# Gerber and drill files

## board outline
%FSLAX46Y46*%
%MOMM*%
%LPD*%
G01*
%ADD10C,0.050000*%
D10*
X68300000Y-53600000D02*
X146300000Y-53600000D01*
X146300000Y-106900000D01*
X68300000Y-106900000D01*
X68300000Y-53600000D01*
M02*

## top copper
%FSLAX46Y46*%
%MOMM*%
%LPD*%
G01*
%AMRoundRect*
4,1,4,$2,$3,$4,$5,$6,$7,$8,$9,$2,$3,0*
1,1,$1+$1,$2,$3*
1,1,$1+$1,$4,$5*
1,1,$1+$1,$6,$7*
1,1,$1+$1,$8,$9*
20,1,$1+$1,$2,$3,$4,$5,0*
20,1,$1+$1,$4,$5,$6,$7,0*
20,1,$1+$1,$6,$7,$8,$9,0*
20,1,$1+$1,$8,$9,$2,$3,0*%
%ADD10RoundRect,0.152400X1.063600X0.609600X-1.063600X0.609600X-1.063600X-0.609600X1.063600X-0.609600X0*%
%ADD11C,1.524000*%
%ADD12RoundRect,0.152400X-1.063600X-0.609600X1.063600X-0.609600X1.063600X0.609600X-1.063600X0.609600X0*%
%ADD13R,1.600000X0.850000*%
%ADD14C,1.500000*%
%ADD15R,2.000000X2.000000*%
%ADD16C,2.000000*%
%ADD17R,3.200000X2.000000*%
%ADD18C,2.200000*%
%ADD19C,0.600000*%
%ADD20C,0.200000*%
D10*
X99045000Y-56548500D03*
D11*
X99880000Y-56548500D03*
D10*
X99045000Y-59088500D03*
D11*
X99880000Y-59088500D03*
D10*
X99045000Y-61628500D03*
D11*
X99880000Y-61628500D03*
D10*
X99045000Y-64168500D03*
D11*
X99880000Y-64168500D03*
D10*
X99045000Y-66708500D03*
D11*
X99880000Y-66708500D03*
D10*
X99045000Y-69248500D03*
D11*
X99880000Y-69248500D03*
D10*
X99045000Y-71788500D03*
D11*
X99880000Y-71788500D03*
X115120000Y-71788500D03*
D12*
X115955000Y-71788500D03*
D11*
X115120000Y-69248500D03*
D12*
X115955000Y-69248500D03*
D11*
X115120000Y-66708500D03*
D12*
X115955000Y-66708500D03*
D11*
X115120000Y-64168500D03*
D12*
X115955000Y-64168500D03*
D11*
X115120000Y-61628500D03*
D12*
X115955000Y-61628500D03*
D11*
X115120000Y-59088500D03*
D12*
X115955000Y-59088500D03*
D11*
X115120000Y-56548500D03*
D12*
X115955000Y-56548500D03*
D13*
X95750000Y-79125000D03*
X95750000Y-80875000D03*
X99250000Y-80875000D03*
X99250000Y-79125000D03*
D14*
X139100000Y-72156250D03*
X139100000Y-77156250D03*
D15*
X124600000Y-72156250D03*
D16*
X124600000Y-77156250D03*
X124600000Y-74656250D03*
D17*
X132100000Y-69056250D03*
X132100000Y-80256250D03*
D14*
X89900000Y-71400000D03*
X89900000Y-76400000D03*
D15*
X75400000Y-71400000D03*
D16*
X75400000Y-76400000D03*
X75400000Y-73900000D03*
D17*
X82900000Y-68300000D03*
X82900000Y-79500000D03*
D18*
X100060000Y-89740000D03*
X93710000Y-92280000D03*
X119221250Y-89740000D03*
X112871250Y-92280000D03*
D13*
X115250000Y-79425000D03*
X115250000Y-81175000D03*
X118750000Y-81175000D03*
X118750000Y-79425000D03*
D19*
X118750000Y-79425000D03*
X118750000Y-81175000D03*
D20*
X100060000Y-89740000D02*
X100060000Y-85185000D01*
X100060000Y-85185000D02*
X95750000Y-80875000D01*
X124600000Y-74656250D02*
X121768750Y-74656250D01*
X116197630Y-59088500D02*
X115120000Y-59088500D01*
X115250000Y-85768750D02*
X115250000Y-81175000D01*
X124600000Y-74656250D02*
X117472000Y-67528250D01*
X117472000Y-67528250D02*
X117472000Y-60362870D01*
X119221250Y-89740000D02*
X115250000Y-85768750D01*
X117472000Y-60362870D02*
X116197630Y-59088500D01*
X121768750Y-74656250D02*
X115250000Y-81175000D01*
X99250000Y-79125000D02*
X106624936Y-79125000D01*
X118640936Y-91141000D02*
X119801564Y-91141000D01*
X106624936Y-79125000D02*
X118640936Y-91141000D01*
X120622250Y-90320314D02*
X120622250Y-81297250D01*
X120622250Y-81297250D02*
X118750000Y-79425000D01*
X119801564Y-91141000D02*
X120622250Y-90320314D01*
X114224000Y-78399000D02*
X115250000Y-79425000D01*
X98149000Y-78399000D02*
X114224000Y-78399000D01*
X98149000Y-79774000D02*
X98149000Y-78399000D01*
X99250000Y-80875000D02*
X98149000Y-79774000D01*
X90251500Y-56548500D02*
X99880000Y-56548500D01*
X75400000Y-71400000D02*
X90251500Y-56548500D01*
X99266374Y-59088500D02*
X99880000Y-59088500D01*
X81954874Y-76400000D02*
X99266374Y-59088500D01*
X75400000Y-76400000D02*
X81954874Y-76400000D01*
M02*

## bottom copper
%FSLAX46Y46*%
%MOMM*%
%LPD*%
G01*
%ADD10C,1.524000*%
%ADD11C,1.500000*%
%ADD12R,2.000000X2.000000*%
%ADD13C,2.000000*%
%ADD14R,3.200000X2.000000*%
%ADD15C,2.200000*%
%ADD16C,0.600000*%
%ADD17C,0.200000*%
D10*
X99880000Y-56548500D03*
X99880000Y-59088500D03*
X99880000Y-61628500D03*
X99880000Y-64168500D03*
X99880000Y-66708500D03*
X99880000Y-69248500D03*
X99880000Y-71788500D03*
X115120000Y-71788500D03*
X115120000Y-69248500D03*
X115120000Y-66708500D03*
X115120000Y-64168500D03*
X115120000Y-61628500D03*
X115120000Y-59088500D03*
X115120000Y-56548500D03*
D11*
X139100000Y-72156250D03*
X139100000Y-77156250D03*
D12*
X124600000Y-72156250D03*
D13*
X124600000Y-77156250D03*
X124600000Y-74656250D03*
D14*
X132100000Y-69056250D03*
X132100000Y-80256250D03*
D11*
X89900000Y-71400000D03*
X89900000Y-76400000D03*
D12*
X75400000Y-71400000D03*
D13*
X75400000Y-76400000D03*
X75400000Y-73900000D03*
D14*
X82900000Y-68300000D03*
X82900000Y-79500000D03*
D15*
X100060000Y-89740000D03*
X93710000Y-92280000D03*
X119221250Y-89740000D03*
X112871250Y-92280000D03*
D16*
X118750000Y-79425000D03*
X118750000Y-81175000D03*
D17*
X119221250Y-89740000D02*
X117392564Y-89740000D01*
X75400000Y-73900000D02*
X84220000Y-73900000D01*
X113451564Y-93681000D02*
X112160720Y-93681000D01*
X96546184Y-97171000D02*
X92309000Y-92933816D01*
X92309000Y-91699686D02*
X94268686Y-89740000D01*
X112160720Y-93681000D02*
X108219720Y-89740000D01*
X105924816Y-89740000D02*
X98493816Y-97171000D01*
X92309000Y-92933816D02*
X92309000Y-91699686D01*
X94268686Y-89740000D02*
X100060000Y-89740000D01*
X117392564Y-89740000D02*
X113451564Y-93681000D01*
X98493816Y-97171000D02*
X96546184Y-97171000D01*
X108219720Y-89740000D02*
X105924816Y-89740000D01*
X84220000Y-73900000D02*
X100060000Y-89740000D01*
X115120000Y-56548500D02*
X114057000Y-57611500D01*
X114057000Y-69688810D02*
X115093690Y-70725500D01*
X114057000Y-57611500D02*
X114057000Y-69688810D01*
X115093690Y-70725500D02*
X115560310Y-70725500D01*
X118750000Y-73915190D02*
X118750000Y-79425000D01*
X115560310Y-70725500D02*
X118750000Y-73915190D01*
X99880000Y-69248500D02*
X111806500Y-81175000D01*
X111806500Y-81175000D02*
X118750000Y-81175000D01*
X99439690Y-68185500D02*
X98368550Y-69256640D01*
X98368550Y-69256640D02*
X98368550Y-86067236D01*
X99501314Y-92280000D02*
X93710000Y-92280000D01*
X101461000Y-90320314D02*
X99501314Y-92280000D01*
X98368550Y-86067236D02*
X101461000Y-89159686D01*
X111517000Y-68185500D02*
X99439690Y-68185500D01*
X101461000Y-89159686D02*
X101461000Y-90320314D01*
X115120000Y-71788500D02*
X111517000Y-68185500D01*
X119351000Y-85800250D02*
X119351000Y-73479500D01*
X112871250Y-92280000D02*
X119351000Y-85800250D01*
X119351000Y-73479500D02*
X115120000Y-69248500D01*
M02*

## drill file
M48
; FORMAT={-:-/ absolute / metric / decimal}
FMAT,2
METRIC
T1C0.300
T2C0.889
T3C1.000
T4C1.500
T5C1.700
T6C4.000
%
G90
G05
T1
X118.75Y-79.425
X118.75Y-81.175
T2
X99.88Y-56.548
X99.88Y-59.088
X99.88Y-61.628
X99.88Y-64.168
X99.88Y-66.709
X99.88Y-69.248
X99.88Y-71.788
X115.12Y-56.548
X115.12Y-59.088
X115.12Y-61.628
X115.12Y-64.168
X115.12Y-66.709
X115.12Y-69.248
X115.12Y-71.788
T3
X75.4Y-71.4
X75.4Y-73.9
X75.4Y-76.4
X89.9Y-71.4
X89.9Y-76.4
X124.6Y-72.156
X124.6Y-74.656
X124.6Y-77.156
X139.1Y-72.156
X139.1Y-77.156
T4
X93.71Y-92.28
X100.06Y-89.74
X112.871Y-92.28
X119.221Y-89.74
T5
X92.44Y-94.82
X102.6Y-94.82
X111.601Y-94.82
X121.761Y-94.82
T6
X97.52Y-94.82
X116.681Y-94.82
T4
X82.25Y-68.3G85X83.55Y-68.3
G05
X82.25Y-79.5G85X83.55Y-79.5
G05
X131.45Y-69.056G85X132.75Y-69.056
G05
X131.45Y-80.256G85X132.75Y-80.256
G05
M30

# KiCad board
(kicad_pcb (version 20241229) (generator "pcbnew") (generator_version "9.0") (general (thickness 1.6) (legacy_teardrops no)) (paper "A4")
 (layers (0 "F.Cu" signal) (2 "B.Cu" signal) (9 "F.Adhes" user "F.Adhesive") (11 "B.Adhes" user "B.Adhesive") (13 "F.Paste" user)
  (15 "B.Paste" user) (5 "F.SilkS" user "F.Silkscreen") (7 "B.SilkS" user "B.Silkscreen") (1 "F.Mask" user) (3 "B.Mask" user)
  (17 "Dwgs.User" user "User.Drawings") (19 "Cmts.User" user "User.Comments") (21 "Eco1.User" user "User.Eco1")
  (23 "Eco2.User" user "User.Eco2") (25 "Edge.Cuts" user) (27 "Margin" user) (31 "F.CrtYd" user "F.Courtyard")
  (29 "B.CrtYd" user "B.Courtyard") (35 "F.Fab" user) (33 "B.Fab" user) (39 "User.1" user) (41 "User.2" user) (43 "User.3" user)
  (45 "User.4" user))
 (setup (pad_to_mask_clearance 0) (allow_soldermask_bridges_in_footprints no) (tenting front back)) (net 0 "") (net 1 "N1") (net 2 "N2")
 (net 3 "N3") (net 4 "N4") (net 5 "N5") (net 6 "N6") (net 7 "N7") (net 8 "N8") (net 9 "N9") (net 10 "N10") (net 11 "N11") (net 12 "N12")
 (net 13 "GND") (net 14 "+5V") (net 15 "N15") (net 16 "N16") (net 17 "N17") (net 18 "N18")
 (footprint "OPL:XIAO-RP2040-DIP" (layer "F.Cu") (at 107.5 64.1685)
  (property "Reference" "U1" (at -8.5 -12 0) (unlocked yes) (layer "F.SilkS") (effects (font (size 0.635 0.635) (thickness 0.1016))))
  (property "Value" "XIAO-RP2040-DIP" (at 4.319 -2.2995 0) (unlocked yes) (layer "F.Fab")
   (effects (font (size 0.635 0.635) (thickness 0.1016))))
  (pad "1" smd roundrect (at -8.455 -7.62 180) (size 2.432 1.524) (layers "F.Cu" "F.Mask") (roundrect_rratio 0.1) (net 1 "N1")
   (thermal_bridge_angle 45))
  (pad "1" thru_hole circle (at -7.62 -7.62 180) (size 1.524 1.524) (drill 0.889) (layers "*.Cu" "*.Mask") (remove_unused_layers no)
   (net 1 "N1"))
  (pad "2" smd roundrect (at -8.455 -5.08 180) (size 2.432 1.524) (layers "F.Cu" "F.Mask") (roundrect_rratio 0.1) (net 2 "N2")
   (thermal_bridge_angle 45))
  (pad "2" thru_hole circle (at -7.62 -5.08 180) (size 1.524 1.524) (drill 0.889) (layers "*.Cu" "*.Mask") (remove_unused_layers no)
   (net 2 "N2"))
  (pad "3" smd roundrect (at -8.455 -2.54 180) (size 2.432 1.524) (layers "F.Cu" "F.Mask") (roundrect_rratio 0.1) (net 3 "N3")
   (thermal_bridge_angle 45))
  (pad "3" thru_hole circle (at -7.62 -2.54 180) (size 1.524 1.524) (drill 0.889) (layers "*.Cu" "*.Mask") (remove_unused_layers no)
   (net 3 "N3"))
  (pad "4" smd roundrect (at -8.455 0 180) (size 2.432 1.524) (layers "F.Cu" "F.Mask") (roundrect_rratio 0.1) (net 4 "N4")
   (thermal_bridge_angle 45))
  (pad "4" thru_hole circle (at -7.62 0 180) (size 1.524 1.524) (drill 0.889) (layers "*.Cu" "*.Mask") (remove_unused_layers no)
   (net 4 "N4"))
  (pad "5" smd roundrect (at -8.455 2.54 180) (size 2.432 1.524) (layers "F.Cu" "F.Mask") (roundrect_rratio 0.1) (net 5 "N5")
   (thermal_bridge_angle 45))
  (pad "5" thru_hole circle (at -7.62 2.54 180) (size 1.524 1.524) (drill 0.889) (layers "*.Cu" "*.Mask") (remove_unused_layers no)
   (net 5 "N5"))
  (pad "6" smd roundrect (at -8.455 5.08 180) (size 2.432 1.524) (layers "F.Cu" "F.Mask") (roundrect_rratio 0.1) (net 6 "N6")
   (thermal_bridge_angle 45))
  (pad "6" thru_hole circle (at -7.62 5.08 180) (size 1.524 1.524) (drill 0.889) (layers "*.Cu" "*.Mask") (remove_unused_layers no)
   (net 6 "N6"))
  (pad "7" smd roundrect (at -8.455 7.62 180) (size 2.432 1.524) (layers "F.Cu" "F.Mask") (roundrect_rratio 0.1) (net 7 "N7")
   (thermal_bridge_angle 45))
  (pad "7" thru_hole circle (at -7.62 7.62 180) (size 1.524 1.524) (drill 0.889) (layers "*.Cu" "*.Mask") (remove_unused_layers no)
   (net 7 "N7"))
  (pad "8" thru_hole circle (at 7.62 7.62) (size 1.524 1.524) (drill 0.889) (layers "*.Cu" "*.Mask") (remove_unused_layers no) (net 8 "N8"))
  (pad "8" smd roundrect (at 8.455 7.62) (size 2.432 1.524) (layers "F.Cu" "F.Mask") (roundrect_rratio 0.1) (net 8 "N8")
   (thermal_bridge_angle 45))
  (pad "9" thru_hole circle (at 7.62 5.08) (size 1.524 1.524) (drill 0.889) (layers "*.Cu" "*.Mask") (remove_unused_layers no) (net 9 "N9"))
  (pad "9" smd roundrect (at 8.455 5.08) (size 2.432 1.524) (layers "F.Cu" "F.Mask") (roundrect_rratio 0.1) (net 9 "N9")
   (thermal_bridge_angle 45))
  (pad "10" thru_hole circle (at 7.62 2.54) (size 1.524 1.524) (drill 0.889) (layers "*.Cu" "*.Mask") (remove_unused_layers no)
   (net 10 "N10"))
  (pad "10" smd roundrect (at 8.455 2.54) (size 2.432 1.524) (layers "F.Cu" "F.Mask") (roundrect_rratio 0.1) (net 10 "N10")
   (thermal_bridge_angle 45))
  (pad "11" thru_hole circle (at 7.62 0) (size 1.524 1.524) (drill 0.889) (layers "*.Cu" "*.Mask") (remove_unused_layers no) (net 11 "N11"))
  (pad "11" smd roundrect (at 8.455 0) (size 2.432 1.524) (layers "F.Cu" "F.Mask") (roundrect_rratio 0.1) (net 11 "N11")
   (thermal_bridge_angle 45))
  (pad "12" thru_hole circle (at 7.62 -2.54) (size 1.524 1.524) (drill 0.889) (layers "*.Cu" "*.Mask") (remove_unused_layers no)
   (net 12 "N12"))
  (pad "12" smd roundrect (at 8.455 -2.54) (size 2.432 1.524) (layers "F.Cu" "F.Mask") (roundrect_rratio 0.1) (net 12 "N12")
   (thermal_bridge_angle 45))
  (pad "13" thru_hole circle (at 7.62 -5.08) (size 1.524 1.524) (drill 0.889) (layers "*.Cu" "*.Mask") (remove_unused_layers no)
   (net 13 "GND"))
  (pad "13" smd roundrect (at 8.455 -5.08) (size 2.432 1.524) (layers "F.Cu" "F.Mask") (roundrect_rratio 0.1) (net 13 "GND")
   (thermal_bridge_angle 45))
  (pad "14" thru_hole circle (at 7.62 -7.62) (size 1.524 1.524) (drill 0.889) (layers "*.Cu" "*.Mask") (remove_unused_layers no)
   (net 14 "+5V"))
  (pad "14" smd roundrect (at 8.455 -7.62) (size 2.432 1.524) (layers "F.Cu" "F.Mask") (roundrect_rratio 0.1) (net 14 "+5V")
   (thermal_bridge_angle 45)))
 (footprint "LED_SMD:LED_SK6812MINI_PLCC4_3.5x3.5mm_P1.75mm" (layer "F.Cu") (at 97.5 80)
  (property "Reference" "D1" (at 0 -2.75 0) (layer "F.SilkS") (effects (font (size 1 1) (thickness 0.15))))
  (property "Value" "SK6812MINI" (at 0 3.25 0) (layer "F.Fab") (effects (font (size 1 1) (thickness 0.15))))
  (pad "1" smd rect (at -1.75 -0.875) (size 1.6 0.85) (layers "F.Cu" "F.Mask" "F.Paste") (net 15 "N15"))
  (pad "2" smd rect (at -1.75 0.875) (size 1.6 0.85) (layers "F.Cu" "F.Mask" "F.Paste") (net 13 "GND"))
  (pad "3" smd rect (at 1.75 0.875) (size 1.6 0.85) (layers "F.Cu" "F.Mask" "F.Paste") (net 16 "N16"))
  (pad "4" smd rect (at 1.75 -0.875) (size 1.6 0.85) (layers "F.Cu" "F.Mask" "F.Paste") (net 14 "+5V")))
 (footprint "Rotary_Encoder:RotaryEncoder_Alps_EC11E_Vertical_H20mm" (layer "F.Cu") (at 124.6 72.15625)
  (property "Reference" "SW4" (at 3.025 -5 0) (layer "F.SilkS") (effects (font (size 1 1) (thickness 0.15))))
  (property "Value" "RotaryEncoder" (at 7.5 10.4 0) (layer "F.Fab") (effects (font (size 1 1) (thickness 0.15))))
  (pad "" thru_hole circle (at 14.5 0) (size 1.5 1.5) (drill 1) (layers "*.Cu" "*.Mask") (remove_unused_layers no))
  (pad "" thru_hole circle (at 14.5 5) (size 1.5 1.5) (drill 1) (layers "*.Cu" "*.Mask") (remove_unused_layers no))
  (pad "A" thru_hole rect (at 0 0) (size 2 2) (drill 1) (layers "*.Cu" "*.Mask") (remove_unused_layers no) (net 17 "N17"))
  (pad "B" thru_hole circle (at 0 5) (size 2 2) (drill 1) (layers "*.Cu" "*.Mask") (remove_unused_layers no) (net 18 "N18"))
  (pad "C" thru_hole circle (at 0 2.5) (size 2 2) (drill 1) (layers "*.Cu" "*.Mask") (remove_unused_layers no) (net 13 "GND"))
  (pad "MP" thru_hole rect (at 7.5 -3.1) (size 3.2 2) (drill oval 2.8 1.5) (layers "*.Cu" "*.Mask") (remove_unused_layers no))
  (pad "MP" thru_hole rect (at 7.5 8.1) (size 3.2 2) (drill oval 2.8 1.5) (layers "*.Cu" "*.Mask") (remove_unused_layers no)))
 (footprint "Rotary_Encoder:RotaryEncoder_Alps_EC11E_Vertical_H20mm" (layer "F.Cu") (at 75.4 71.4)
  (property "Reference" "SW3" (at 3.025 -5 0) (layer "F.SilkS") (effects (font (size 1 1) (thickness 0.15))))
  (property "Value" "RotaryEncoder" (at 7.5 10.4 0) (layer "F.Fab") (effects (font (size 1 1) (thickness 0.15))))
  (pad "" thru_hole circle (at 14.5 0) (size 1.5 1.5) (drill 1) (layers "*.Cu" "*.Mask") (remove_unused_layers no))
  (pad "" thru_hole circle (at 14.5 5) (size 1.5 1.5) (drill 1) (layers "*.Cu" "*.Mask") (remove_unused_layers no))
  (pad "A" thru_hole rect (at 0 0) (size 2 2) (drill 1) (layers "*.Cu" "*.Mask") (remove_unused_layers no) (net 1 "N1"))
  (pad "B" thru_hole circle (at 0 5) (size 2 2) (drill 1) (layers "*.Cu" "*.Mask") (remove_unused_layers no) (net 2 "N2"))
  (pad "C" thru_hole circle (at 0 2.5) (size 2 2) (drill 1) (layers "*.Cu" "*.Mask") (remove_unused_layers no) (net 13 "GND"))
  (pad "MP" thru_hole rect (at 7.5 -3.1) (size 3.2 2) (drill oval 2.8 1.5) (layers "*.Cu" "*.Mask") (remove_unused_layers no))
  (pad "MP" thru_hole rect (at 7.5 8.1) (size 3.2 2) (drill oval 2.8 1.5) (layers "*.Cu" "*.Mask") (remove_unused_layers no)))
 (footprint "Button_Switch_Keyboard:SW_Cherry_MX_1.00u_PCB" (layer "F.Cu") (at 100.06 89.74)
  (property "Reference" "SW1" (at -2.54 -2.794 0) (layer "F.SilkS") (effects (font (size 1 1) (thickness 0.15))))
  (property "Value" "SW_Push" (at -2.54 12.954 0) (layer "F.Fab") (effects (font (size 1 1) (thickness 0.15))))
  (pad "" np_thru_hole circle (at -7.62 5.08) (size 1.7 1.7) (drill 1.7) (layers "*.Cu" "*.Mask"))
  (pad "" np_thru_hole circle (at -2.54 5.08) (size 4 4) (drill 4) (layers "*.Cu" "*.Mask"))
  (pad "" np_thru_hole circle (at 2.54 5.08) (size 1.7 1.7) (drill 1.7) (layers "*.Cu" "*.Mask"))
  (pad "1" thru_hole circle (at 0 0) (size 2.2 2.2) (drill 1.5) (layers "*.Cu" "*.Mask") (remove_unused_layers no) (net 13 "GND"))
  (pad "2" thru_hole circle (at -6.35 2.54) (size 2.2 2.2) (drill 1.5) (layers "*.Cu" "*.Mask") (remove_unused_layers no) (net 8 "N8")))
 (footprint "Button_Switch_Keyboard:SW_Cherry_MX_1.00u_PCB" (layer "F.Cu") (at 119.22125 89.74)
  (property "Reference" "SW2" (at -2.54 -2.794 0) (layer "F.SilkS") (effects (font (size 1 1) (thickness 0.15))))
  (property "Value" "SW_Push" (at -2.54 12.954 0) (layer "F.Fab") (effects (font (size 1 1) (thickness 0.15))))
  (pad "" np_thru_hole circle (at -7.62 5.08) (size 1.7 1.7) (drill 1.7) (layers "*.Cu" "*.Mask"))
  (pad "" np_thru_hole circle (at -2.54 5.08) (size 4 4) (drill 4) (layers "*.Cu" "*.Mask"))
  (pad "" np_thru_hole circle (at 2.54 5.08) (size 1.7 1.7) (drill 1.7) (layers "*.Cu" "*.Mask"))
  (pad "1" thru_hole circle (at 0 0) (size 2.2 2.2) (drill 1.5) (layers "*.Cu" "*.Mask") (remove_unused_layers no) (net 13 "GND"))
  (pad "2" thru_hole circle (at -6.35 2.54) (size 2.2 2.2) (drill 1.5) (layers "*.Cu" "*.Mask") (remove_unused_layers no) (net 9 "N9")))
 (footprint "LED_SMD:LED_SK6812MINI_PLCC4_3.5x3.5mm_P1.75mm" (layer "F.Cu") (at 117 80.3)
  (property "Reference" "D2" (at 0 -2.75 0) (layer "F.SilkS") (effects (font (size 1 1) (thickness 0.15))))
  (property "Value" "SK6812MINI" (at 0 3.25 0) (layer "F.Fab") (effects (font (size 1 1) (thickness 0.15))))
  (pad "1" smd rect (at -1.75 -0.875) (size 1.6 0.85) (layers "F.Cu" "F.Mask" "F.Paste") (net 16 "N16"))
  (pad "2" smd rect (at -1.75 0.875) (size 1.6 0.85) (layers "F.Cu" "F.Mask" "F.Paste") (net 13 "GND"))
  (pad "3" smd rect (at 1.75 0.875) (size 1.6 0.85) (layers "F.Cu" "F.Mask" "F.Paste") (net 6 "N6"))
  (pad "4" smd rect (at 1.75 -0.875) (size 1.6 0.85) (layers "F.Cu" "F.Mask" "F.Paste") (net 14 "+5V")))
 (gr_rect (start 68.3 53.6) (end 146.3 106.9) (stroke (width 0.05) (type default)) (fill no) (layer "Edge.Cuts"))
 (segment (start 100.06 89.74) (end 100.06 85.185) (width 0.2) (layer "F.Cu") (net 13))
 (segment (start 100.06 85.185) (end 95.75 80.875) (width 0.2) (layer "F.Cu") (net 13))
 (segment (start 124.6 74.65625) (end 121.76875 74.65625) (width 0.2) (layer "F.Cu") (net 13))
 (segment (start 116.19763 59.0885) (end 115.12 59.0885) (width 0.2) (layer "F.Cu") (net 13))
 (segment (start 115.25 85.76875) (end 115.25 81.175) (width 0.2) (layer "F.Cu") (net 13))
 (segment (start 124.6 74.65625) (end 117.472 67.52825) (width 0.2) (layer "F.Cu") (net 13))
 (segment (start 117.472 67.52825) (end 117.472 60.36287) (width 0.2) (layer "F.Cu") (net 13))
 (segment (start 119.22125 89.74) (end 115.25 85.76875) (width 0.2) (layer "F.Cu") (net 13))
 (segment (start 117.472 60.36287) (end 116.19763 59.0885) (width 0.2) (layer "F.Cu") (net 13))
 (segment (start 121.76875 74.65625) (end 115.25 81.175) (width 0.2) (layer "F.Cu") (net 13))
 (segment (start 119.22125 89.74) (end 117.392564 89.74) (width 0.2) (layer "B.Cu") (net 13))
 (segment (start 75.4 73.9) (end 84.22 73.9) (width 0.2) (layer "B.Cu") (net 13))
 (segment (start 113.451564 93.681) (end 112.16072 93.681) (width 0.2) (layer "B.Cu") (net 13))
 (segment (start 96.546184 97.171) (end 92.309 92.933816) (width 0.2) (layer "B.Cu") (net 13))
 (segment (start 92.309 91.699686) (end 94.268686 89.74) (width 0.2) (layer "B.Cu") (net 13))
 (segment (start 112.16072 93.681) (end 108.21972 89.74) (width 0.2) (layer "B.Cu") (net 13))
 (segment (start 105.924816 89.74) (end 98.493816 97.171) (width 0.2) (layer "B.Cu") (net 13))
 (segment (start 92.309 92.933816) (end 92.309 91.699686) (width 0.2) (layer "B.Cu") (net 13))
 (segment (start 94.268686 89.74) (end 100.06 89.74) (width 0.2) (layer "B.Cu") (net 13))
 (segment (start 117.392564 89.74) (end 113.451564 93.681) (width 0.2) (layer "B.Cu") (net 13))
 (segment (start 98.493816 97.171) (end 96.546184 97.171) (width 0.2) (layer "B.Cu") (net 13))
 (segment (start 108.21972 89.74) (end 105.924816 89.74) (width 0.2) (layer "B.Cu") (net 13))
 (segment (start 84.22 73.9) (end 100.06 89.74) (width 0.2) (layer "B.Cu") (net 13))
 (segment (start 99.25 79.125) (end 106.624936 79.125) (width 0.2) (layer "F.Cu") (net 14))
 (segment (start 118.640936 91.141) (end 119.801564 91.141) (width 0.2) (layer "F.Cu") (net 14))
 (segment (start 106.624936 79.125) (end 118.640936 91.141) (width 0.2) (layer "F.Cu") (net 14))
 (segment (start 120.62225 90.320314) (end 120.62225 81.29725) (width 0.2) (layer "F.Cu") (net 14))
 (segment (start 120.62225 81.29725) (end 118.75 79.425) (width 0.2) (layer "F.Cu") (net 14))
 (segment (start 119.801564 91.141) (end 120.62225 90.320314) (width 0.2) (layer "F.Cu") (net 14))
 (via (at 118.75 79.425) (size 0.6) (drill 0.3) (layers "F.Cu" "B.Cu") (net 14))
 (segment (start 115.12 56.5485) (end 114.057 57.6115) (width 0.2) (layer "B.Cu") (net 14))
 (segment (start 114.057 69.68881) (end 115.09369 70.7255) (width 0.2) (layer "B.Cu") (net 14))
 (segment (start 114.057 57.6115) (end 114.057 69.68881) (width 0.2) (layer "B.Cu") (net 14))
 (segment (start 115.09369 70.7255) (end 115.56031 70.7255) (width 0.2) (layer "B.Cu") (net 14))
 (segment (start 118.75 73.91519) (end 118.75 79.425) (width 0.2) (layer "B.Cu") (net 14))
 (segment (start 115.56031 70.7255) (end 118.75 73.91519) (width 0.2) (layer "B.Cu") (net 14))
 (segment (start 114.224 78.399) (end 115.25 79.425) (width 0.2) (layer "F.Cu") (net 16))
 (segment (start 98.149 78.399) (end 114.224 78.399) (width 0.2) (layer "F.Cu") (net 16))
 (segment (start 98.149 79.774) (end 98.149 78.399) (width 0.2) (layer "F.Cu") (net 16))
 (segment (start 99.25 80.875) (end 98.149 79.774) (width 0.2) (layer "F.Cu") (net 16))
 (via (at 118.75 81.175) (size 0.6) (drill 0.3) (layers "F.Cu" "B.Cu") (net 6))
 (segment (start 99.88 69.2485) (end 111.8065 81.175) (width 0.2) (layer "B.Cu") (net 6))
 (segment (start 111.8065 81.175) (end 118.75 81.175) (width 0.2) (layer "B.Cu") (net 6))
 (segment (start 99.43969 68.1855) (end 98.36855 69.25664) (width 0.2) (layer "B.Cu") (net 8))
 (segment (start 98.36855 69.25664) (end 98.36855 86.067236) (width 0.2) (layer "B.Cu") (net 8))
 (segment (start 99.501314 92.28) (end 93.71 92.28) (width 0.2) (layer "B.Cu") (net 8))
 (segment (start 101.461 90.320314) (end 99.501314 92.28) (width 0.2) (layer "B.Cu") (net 8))
 (segment (start 98.36855 86.067236) (end 101.461 89.159686) (width 0.2) (layer "B.Cu") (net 8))
 (segment (start 111.517 68.1855) (end 99.43969 68.1855) (width 0.2) (layer "B.Cu") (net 8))
 (segment (start 101.461 89.159686) (end 101.461 90.320314) (width 0.2) (layer "B.Cu") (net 8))
 (segment (start 115.12 71.7885) (end 111.517 68.1855) (width 0.2) (layer "B.Cu") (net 8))
 (segment (start 119.351 85.80025) (end 119.351 73.4795) (width 0.2) (layer "B.Cu") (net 9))
 (segment (start 112.87125 92.28) (end 119.351 85.80025) (width 0.2) (layer "B.Cu") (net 9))
 (segment (start 119.351 73.4795) (end 115.12 69.2485) (width 0.2) (layer "B.Cu") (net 9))
 (segment (start 90.2515 56.5485) (end 99.88 56.5485) (width 0.2) (layer "F.Cu") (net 1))
 (segment (start 75.4 71.4) (end 90.2515 56.5485) (width 0.2) (layer "F.Cu") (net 1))
 (segment (start 99.266374 59.0885) (end 99.88 59.0885) (width 0.2) (layer "F.Cu") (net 2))
 (segment (start 81.954874 76.4) (end 99.266374 59.0885) (width 0.2) (layer "F.Cu") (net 2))
 (segment (start 75.4 76.4) (end 81.954874 76.4) (width 0.2) (layer "F.Cu") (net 2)))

